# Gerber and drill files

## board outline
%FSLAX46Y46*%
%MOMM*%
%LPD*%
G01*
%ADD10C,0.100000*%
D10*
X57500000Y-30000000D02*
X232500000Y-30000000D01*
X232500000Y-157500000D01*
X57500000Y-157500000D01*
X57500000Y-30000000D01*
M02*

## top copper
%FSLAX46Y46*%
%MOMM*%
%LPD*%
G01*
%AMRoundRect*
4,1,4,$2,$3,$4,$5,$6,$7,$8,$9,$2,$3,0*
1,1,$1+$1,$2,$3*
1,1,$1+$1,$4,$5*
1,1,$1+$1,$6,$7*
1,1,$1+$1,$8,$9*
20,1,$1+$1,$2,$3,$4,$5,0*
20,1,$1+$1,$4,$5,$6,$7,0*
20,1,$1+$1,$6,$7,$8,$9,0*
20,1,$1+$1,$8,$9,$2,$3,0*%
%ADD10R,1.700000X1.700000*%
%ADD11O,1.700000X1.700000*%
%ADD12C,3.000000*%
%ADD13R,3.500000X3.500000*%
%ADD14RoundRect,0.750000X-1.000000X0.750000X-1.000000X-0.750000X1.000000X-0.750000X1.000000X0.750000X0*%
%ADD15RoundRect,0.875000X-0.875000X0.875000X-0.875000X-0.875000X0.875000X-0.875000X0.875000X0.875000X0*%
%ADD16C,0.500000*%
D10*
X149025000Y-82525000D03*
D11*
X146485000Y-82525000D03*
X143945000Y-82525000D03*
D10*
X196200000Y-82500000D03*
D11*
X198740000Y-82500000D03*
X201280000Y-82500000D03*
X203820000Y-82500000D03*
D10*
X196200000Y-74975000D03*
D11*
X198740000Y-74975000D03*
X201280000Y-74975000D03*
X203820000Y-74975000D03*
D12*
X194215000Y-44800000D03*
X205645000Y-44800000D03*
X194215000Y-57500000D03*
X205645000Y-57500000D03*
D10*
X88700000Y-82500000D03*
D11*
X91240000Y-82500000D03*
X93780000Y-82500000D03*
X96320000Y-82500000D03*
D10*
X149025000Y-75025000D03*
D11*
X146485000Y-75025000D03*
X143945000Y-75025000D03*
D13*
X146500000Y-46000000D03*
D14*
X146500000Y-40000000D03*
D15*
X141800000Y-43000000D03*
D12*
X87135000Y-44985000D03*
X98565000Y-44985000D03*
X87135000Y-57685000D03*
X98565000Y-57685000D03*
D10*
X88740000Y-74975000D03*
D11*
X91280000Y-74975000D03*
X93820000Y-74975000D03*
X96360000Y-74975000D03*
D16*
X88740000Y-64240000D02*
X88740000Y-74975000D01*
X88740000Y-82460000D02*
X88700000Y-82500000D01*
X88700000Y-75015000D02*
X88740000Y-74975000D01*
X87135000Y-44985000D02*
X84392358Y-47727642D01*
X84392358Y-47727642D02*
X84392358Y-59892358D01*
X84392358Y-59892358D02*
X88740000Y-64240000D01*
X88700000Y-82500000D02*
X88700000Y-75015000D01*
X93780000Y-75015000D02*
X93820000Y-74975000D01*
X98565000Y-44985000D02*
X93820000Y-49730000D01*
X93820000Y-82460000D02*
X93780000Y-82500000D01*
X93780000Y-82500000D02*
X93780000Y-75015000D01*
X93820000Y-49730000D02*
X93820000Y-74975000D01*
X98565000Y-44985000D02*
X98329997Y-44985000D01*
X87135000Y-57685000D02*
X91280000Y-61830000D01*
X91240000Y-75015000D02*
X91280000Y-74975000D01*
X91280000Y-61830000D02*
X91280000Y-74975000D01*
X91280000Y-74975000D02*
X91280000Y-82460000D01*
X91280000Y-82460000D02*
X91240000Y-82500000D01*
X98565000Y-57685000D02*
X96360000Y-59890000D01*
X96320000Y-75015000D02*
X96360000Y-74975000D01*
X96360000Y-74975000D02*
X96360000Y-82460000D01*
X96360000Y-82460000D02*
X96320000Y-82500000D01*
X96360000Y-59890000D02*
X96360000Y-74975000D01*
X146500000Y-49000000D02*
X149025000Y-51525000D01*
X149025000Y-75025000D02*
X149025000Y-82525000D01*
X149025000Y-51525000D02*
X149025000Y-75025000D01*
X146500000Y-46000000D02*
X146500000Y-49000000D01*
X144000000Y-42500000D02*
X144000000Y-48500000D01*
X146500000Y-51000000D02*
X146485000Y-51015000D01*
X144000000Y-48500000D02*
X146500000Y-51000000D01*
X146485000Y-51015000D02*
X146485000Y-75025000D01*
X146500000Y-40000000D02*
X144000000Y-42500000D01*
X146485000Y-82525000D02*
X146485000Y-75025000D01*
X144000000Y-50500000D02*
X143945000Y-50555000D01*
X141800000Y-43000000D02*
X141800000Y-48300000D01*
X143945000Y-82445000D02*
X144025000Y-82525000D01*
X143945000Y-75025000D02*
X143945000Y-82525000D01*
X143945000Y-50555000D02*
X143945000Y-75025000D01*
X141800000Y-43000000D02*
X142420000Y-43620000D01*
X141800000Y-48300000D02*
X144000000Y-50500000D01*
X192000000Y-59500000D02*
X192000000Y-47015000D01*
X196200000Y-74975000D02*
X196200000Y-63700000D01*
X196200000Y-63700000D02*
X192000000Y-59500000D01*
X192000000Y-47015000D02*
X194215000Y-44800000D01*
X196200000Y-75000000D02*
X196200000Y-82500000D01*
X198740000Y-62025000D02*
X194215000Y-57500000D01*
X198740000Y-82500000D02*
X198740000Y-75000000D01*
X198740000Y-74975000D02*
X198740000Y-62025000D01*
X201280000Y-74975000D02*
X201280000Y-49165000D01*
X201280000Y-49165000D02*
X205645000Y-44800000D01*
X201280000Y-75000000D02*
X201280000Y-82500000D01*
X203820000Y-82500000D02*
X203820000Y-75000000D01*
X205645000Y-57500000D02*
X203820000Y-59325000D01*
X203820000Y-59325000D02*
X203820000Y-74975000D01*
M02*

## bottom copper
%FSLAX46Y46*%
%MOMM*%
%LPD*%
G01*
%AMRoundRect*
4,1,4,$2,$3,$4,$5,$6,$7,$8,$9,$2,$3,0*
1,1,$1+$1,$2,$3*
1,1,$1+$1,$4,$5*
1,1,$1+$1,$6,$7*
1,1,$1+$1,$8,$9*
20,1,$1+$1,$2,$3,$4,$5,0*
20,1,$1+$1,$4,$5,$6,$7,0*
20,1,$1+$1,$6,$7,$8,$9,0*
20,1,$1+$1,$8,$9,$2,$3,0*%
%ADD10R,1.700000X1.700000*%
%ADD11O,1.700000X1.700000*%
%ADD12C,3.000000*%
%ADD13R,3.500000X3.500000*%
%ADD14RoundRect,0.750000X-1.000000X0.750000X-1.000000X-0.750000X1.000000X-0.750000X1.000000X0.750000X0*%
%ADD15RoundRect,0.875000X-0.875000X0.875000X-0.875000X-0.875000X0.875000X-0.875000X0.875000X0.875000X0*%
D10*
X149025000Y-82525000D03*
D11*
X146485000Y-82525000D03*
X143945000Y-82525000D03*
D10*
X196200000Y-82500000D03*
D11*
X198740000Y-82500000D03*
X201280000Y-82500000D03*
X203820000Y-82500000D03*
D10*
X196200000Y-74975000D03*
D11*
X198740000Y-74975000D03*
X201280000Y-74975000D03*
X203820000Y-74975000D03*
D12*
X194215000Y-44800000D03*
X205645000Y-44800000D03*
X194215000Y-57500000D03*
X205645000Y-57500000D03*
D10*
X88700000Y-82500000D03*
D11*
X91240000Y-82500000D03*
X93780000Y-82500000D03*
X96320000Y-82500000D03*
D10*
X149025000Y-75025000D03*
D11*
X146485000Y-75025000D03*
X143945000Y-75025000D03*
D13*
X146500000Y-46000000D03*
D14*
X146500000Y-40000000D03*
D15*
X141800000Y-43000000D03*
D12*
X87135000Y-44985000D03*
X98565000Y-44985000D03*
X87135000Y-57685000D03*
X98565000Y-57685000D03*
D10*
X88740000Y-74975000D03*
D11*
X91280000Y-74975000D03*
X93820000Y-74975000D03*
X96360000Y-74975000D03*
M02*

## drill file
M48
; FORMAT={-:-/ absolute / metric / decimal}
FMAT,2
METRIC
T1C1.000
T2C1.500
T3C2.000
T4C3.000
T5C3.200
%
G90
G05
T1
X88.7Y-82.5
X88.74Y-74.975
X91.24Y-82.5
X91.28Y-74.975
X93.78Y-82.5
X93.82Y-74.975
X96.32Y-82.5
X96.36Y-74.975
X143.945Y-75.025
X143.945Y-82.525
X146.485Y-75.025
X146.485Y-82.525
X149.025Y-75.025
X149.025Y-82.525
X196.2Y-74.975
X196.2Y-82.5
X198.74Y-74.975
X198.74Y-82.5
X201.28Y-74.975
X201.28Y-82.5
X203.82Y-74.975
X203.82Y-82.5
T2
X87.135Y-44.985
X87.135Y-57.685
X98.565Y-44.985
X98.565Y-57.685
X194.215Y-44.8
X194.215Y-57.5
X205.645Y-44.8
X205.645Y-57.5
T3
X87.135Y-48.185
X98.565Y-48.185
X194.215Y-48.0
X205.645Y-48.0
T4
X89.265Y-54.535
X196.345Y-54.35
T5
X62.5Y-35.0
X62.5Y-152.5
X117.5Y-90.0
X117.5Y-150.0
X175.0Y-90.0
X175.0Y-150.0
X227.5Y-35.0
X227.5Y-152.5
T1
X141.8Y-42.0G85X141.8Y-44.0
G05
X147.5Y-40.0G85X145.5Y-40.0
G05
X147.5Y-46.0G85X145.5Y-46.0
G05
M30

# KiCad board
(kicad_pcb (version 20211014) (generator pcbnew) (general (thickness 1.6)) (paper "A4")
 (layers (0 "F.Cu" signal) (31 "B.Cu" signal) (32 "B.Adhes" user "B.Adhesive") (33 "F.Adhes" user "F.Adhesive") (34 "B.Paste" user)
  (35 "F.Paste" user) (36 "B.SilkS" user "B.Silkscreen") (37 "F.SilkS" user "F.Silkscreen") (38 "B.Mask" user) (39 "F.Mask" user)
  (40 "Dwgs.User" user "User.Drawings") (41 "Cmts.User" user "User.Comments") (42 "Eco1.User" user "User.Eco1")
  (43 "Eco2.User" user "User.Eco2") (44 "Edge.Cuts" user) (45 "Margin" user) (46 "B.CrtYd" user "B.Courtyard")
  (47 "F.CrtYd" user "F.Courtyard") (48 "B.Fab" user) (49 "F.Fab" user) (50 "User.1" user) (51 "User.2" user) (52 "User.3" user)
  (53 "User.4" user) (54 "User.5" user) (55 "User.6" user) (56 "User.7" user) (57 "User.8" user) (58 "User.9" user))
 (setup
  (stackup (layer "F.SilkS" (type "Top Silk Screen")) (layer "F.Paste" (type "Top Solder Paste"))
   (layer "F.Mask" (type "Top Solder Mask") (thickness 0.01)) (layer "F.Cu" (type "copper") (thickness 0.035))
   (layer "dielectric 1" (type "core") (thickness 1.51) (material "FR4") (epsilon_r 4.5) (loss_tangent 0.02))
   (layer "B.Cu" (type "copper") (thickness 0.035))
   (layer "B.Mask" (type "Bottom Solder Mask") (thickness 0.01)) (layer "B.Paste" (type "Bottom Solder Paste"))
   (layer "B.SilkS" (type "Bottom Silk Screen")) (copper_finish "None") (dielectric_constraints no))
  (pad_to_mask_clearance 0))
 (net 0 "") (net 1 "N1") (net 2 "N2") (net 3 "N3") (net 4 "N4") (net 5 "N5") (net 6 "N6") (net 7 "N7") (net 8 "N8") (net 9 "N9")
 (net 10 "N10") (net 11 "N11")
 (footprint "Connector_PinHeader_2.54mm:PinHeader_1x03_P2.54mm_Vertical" (layer "F.Cu") (at 149.025 82.525 -90)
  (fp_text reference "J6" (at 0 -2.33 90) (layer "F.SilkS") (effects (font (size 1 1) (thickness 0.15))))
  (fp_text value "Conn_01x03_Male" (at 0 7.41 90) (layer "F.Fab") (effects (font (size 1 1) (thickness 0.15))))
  (pad "1" thru_hole rect (at 0 0 270) (size 1.7 1.7) (drill 1) (layers *.Cu *.Mask) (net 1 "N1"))
  (pad "2" thru_hole oval (at 0 2.54 270) (size 1.7 1.7) (drill 1) (layers *.Cu *.Mask) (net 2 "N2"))
  (pad "3" thru_hole oval (at 0 5.08 270) (size 1.7 1.7) (drill 1) (layers *.Cu *.Mask) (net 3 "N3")))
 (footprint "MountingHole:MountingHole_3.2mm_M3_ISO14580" (layer "F.Cu") (at 227.5 152.5)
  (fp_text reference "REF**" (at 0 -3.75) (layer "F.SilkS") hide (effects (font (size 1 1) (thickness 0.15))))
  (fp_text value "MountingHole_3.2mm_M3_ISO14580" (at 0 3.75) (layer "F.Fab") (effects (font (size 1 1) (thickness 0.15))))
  (pad "" np_thru_hole circle (at 0 0) (size 3.2 3.2) (drill 3.2) (layers *.Cu *.Mask)))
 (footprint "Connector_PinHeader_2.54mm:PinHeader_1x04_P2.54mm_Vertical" (layer "F.Cu") (at 196.2 82.5 90)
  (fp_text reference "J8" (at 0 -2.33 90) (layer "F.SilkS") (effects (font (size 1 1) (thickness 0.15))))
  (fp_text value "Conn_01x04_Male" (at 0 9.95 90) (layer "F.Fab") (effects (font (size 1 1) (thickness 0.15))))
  (pad "1" thru_hole rect (at 0 0 90) (size 1.7 1.7) (drill 1) (layers *.Cu *.Mask) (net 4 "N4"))
  (pad "2" thru_hole oval (at 0 2.54 90) (size 1.7 1.7) (drill 1) (layers *.Cu *.Mask) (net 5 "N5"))
  (pad "3" thru_hole oval (at 0 5.08 90) (size 1.7 1.7) (drill 1) (layers *.Cu *.Mask) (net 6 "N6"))
  (pad "4" thru_hole oval (at 0 7.62 90) (size 1.7 1.7) (drill 1) (layers *.Cu *.Mask) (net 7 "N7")))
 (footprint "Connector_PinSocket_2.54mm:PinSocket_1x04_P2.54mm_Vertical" (layer "F.Cu") (at 196.2 74.975 90)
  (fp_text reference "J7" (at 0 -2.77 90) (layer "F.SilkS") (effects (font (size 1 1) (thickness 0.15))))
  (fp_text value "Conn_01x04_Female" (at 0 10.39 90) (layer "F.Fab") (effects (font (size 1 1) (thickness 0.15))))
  (pad "1" thru_hole rect (at 0 0 90) (size 1.7 1.7) (drill 1) (layers *.Cu *.Mask) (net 4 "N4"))
  (pad "2" thru_hole oval (at 0 2.54 90) (size 1.7 1.7) (drill 1) (layers *.Cu *.Mask) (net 5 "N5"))
  (pad "3" thru_hole oval (at 0 5.08 90) (size 1.7 1.7) (drill 1) (layers *.Cu *.Mask) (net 6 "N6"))
  (pad "4" thru_hole oval (at 0 7.62 90) (size 1.7 1.7) (drill 1) (layers *.Cu *.Mask) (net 7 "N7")))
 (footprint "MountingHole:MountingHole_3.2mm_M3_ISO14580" (layer "F.Cu") (at 117.5 150)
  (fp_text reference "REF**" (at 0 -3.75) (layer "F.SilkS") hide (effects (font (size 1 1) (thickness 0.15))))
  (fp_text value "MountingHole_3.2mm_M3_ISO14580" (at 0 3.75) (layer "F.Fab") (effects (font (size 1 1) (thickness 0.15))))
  (pad "" np_thru_hole circle (at 0 0) (size 3.2 3.2) (drill 3.2) (layers *.Cu *.Mask)))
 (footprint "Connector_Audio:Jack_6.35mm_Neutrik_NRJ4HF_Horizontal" (layer "F.Cu") (at 194.215 57.5 90)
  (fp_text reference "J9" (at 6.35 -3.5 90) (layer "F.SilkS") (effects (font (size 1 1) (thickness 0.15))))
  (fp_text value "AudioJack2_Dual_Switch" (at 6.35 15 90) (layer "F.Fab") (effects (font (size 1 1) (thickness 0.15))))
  (pad "" np_thru_hole circle (at 3.15 2.13 90) (size 3 3) (drill 3) (layers *.Cu *.Mask))
  (pad "" np_thru_hole circle (at 9.5 0 90) (size 2 2) (drill 2) (layers *.Cu *.Mask))
  (pad "" np_thru_hole circle (at 9.5 11.43 90) (size 2 2) (drill 2) (layers *.Cu *.Mask))
  (pad "S" thru_hole circle (at 12.7 0 90) (size 3 3) (drill 1.5) (layers *.Cu *.Mask) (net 4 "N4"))
  (pad "SN" thru_hole circle (at 12.7 11.43 90) (size 3 3) (drill 1.5) (layers *.Cu *.Mask) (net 6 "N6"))
  (pad "T" thru_hole circle (at 0 0 90) (size 3 3) (drill 1.5) (layers *.Cu *.Mask) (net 5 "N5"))
  (pad "TN" thru_hole circle (at 0 11.43 90) (size 3 3) (drill 1.5) (layers *.Cu *.Mask) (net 7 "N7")))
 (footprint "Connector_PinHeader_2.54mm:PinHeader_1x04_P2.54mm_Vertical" (layer "F.Cu") (at 88.7 82.5 90)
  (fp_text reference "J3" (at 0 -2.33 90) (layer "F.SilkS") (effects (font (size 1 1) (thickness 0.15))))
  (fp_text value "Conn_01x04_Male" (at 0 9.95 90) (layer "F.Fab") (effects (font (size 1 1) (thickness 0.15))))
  (pad "1" thru_hole rect (at 0 0 90) (size 1.7 1.7) (drill 1) (layers *.Cu *.Mask) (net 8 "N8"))
  (pad "2" thru_hole oval (at 0 2.54 90) (size 1.7 1.7) (drill 1) (layers *.Cu *.Mask) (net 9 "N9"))
  (pad "3" thru_hole oval (at 0 5.08 90) (size 1.7 1.7) (drill 1) (layers *.Cu *.Mask) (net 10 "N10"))
  (pad "4" thru_hole oval (at 0 7.62 90) (size 1.7 1.7) (drill 1) (layers *.Cu *.Mask) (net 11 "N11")))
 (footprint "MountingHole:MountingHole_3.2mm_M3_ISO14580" (layer "F.Cu") (at 117.5 90)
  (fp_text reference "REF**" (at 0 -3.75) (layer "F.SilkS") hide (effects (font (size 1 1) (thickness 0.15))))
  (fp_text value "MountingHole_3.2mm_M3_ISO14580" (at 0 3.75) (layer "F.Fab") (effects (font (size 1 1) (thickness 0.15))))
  (pad "" np_thru_hole circle (at 0 0) (size 3.2 3.2) (drill 3.2) (layers *.Cu *.Mask)))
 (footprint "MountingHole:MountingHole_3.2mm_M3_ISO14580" (layer "F.Cu") (at 62.5 35)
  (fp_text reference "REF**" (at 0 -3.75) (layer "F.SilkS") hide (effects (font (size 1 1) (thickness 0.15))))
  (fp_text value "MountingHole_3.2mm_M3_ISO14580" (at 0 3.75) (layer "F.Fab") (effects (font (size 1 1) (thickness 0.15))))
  (pad "" np_thru_hole circle (at 0 0) (size 3.2 3.2) (drill 3.2) (layers *.Cu *.Mask)))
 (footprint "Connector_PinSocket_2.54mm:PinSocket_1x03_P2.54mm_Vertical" (layer "F.Cu") (at 149.025 75.025 -90)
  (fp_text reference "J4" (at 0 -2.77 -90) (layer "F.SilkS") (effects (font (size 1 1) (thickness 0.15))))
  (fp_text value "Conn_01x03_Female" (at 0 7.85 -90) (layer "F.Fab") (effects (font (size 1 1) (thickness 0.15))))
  (pad "1" thru_hole rect (at 0 0 270) (size 1.7 1.7) (drill 1) (layers *.Cu *.Mask) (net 1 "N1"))
  (pad "2" thru_hole oval (at 0 2.54 270) (size 1.7 1.7) (drill 1) (layers *.Cu *.Mask) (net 2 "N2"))
  (pad "3" thru_hole oval (at 0 5.08 270) (size 1.7 1.7) (drill 1) (layers *.Cu *.Mask) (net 3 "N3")))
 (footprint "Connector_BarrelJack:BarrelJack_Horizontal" (layer "F.Cu") (at 146.5 46 -90)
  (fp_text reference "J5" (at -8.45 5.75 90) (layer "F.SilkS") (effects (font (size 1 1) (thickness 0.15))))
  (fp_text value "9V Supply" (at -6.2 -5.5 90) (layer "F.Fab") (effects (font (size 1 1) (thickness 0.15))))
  (pad "1" thru_hole rect (at 0 0 270) (size 3.5 3.5) (drill oval 1 3) (layers *.Cu *.Mask) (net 1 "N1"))
  (pad "2" thru_hole roundrect (at -6 0 270) (size 3 3.5) (drill oval 1 3) (layers *.Cu *.Mask) (roundrect_rratio 0.25) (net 2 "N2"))
  (pad "3" thru_hole roundrect (at -3 4.7 270) (size 3.5 3.5) (drill oval 3 1) (layers *.Cu *.Mask) (roundrect_rratio 0.25) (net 3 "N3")))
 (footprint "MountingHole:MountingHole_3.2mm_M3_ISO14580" (layer "F.Cu") (at 175 90)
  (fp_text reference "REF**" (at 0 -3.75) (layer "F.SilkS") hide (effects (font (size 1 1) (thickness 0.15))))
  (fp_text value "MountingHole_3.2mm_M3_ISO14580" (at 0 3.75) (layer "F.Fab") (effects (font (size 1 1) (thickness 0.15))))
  (pad "" np_thru_hole circle (at 0 0) (size 3.2 3.2) (drill 3.2) (layers *.Cu *.Mask)))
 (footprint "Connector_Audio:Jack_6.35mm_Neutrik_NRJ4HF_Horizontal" (layer "F.Cu") (at 87.135 57.685 90)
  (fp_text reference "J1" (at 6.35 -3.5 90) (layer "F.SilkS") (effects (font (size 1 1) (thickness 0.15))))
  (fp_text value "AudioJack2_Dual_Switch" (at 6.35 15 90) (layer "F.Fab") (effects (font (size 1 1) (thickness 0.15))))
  (pad "" np_thru_hole circle (at 3.15 2.13 90) (size 3 3) (drill 3) (layers *.Cu *.Mask))
  (pad "" np_thru_hole circle (at 9.5 11.43 90) (size 2 2) (drill 2) (layers *.Cu *.Mask))
  (pad "" np_thru_hole circle (at 9.5 0 90) (size 2 2) (drill 2) (layers *.Cu *.Mask))
  (pad "S" thru_hole circle (at 12.7 0 90) (size 3 3) (drill 1.5) (layers *.Cu *.Mask) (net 8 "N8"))
  (pad "SN" thru_hole circle (at 12.7 11.43 90) (size 3 3) (drill 1.5) (layers *.Cu *.Mask) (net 10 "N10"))
  (pad "T" thru_hole circle (at 0 0 90) (size 3 3) (drill 1.5) (layers *.Cu *.Mask) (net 9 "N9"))
  (pad "TN" thru_hole circle (at 0 11.43 90) (size 3 3) (drill 1.5) (layers *.Cu *.Mask) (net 11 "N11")))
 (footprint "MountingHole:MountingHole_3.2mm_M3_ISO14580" (layer "F.Cu") (at 62.5 152.5)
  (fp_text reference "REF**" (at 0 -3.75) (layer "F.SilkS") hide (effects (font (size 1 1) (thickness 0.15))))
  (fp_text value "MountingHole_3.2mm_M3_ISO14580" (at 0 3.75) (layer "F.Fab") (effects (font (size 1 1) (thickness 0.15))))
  (pad "" np_thru_hole circle (at 0 0) (size 3.2 3.2) (drill 3.2) (layers *.Cu *.Mask)))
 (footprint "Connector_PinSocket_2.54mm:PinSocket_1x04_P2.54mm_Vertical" (layer "F.Cu") (at 88.74 74.975 90)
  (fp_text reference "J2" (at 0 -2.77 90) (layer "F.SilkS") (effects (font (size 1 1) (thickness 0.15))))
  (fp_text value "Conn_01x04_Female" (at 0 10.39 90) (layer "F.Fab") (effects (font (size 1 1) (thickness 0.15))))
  (pad "1" thru_hole rect (at 0 0 90) (size 1.7 1.7) (drill 1) (layers *.Cu *.Mask) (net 8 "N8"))
  (pad "2" thru_hole oval (at 0 2.54 90) (size 1.7 1.7) (drill 1) (layers *.Cu *.Mask) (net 9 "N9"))
  (pad "3" thru_hole oval (at 0 5.08 90) (size 1.7 1.7) (drill 1) (layers *.Cu *.Mask) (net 10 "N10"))
  (pad "4" thru_hole oval (at 0 7.62 90) (size 1.7 1.7) (drill 1) (layers *.Cu *.Mask) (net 11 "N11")))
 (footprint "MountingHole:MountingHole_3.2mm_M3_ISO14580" (layer "F.Cu") (at 175 150)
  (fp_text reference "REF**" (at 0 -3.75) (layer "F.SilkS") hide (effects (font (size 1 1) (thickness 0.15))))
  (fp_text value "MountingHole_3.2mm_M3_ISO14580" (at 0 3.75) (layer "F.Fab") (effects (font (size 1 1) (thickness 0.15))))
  (pad "" np_thru_hole circle (at 0 0) (size 3.2 3.2) (drill 3.2) (layers *.Cu *.Mask)))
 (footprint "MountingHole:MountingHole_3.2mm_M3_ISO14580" (layer "F.Cu") (at 227.5 35)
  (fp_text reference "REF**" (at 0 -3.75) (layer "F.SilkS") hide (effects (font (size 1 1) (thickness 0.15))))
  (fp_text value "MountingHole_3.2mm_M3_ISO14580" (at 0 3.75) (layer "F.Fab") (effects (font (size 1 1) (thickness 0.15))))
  (pad "" np_thru_hole circle (at 0 0) (size 3.2 3.2) (drill 3.2) (layers *.Cu *.Mask)))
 (gr_rect (start 57.5 30) (end 232.5 157.5) (layer "Edge.Cuts") (width 0.1) (fill none))
 (segment (start 88.74 64.24) (end 88.74 74.975) (width 0.5) (layer "F.Cu") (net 8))
 (segment (start 88.74 82.46) (end 88.7 82.5) (width 0.5) (layer "F.Cu") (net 8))
 (segment (start 88.7 75.015) (end 88.74 74.975) (width 0.5) (layer "F.Cu") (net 8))
 (segment (start 87.135 44.985) (end 84.392358 47.727642) (width 0.5) (layer "F.Cu") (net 8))
 (segment (start 84.392358 47.727642) (end 84.392358 59.892358) (width 0.5) (layer "F.Cu") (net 8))
 (segment (start 84.392358 59.892358) (end 88.74 64.24) (width 0.5) (layer "F.Cu") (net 8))
 (segment (start 88.7 82.5) (end 88.7 75.015) (width 0.5) (layer "F.Cu") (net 8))
 (segment (start 93.78 75.015) (end 93.82 74.975) (width 0.5) (layer "F.Cu") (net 10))
 (segment (start 98.565 44.985) (end 93.82 49.73) (width 0.5) (layer "F.Cu") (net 10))
 (segment (start 93.82 82.46) (end 93.78 82.5) (width 0.5) (layer "F.Cu") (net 10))
 (segment (start 93.78 82.5) (end 93.78 75.015) (width 0.5) (layer "F.Cu") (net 10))
 (segment (start 93.82 49.73) (end 93.82 74.975) (width 0.5) (layer "F.Cu") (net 10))
 (segment (start 98.565 44.985) (end 98.329997 44.985) (width 0.5) (layer "F.Cu") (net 10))
 (segment (start 87.135 57.685) (end 91.28 61.83) (width 0.5) (layer "F.Cu") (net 9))
 (segment (start 91.24 75.015) (end 91.28 74.975) (width 0.5) (layer "F.Cu") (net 9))
 (segment (start 91.28 61.83) (end 91.28 74.975) (width 0.5) (layer "F.Cu") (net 9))
 (segment (start 91.28 74.975) (end 91.28 82.46) (width 0.5) (layer "F.Cu") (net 9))
 (segment (start 91.28 82.46) (end 91.24 82.5) (width 0.5) (layer "F.Cu") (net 9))
 (segment (start 98.565 57.685) (end 96.36 59.89) (width 0.5) (layer "F.Cu") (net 11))
 (segment (start 96.32 75.015) (end 96.36 74.975) (width 0.5) (layer "F.Cu") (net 11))
 (segment (start 96.36 74.975) (end 96.36 82.46) (width 0.5) (layer "F.Cu") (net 11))
 (segment (start 96.36 82.46) (end 96.32 82.5) (width 0.5) (layer "F.Cu") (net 11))
 (segment (start 96.36 59.89) (end 96.36 74.975) (width 0.5) (layer "F.Cu") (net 11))
 (segment (start 146.5 49) (end 149.025 51.525) (width 0.5) (layer "F.Cu") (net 1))
 (segment (start 149.025 75.025) (end 149.025 82.525) (width 0.5) (layer "F.Cu") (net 1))
 (segment (start 149.025 51.525) (end 149.025 75.025) (width 0.5) (layer "F.Cu") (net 1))
 (segment (start 146.5 46) (end 146.5 49) (width 0.5) (layer "F.Cu") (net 1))
 (segment (start 144 42.5) (end 144 48.5) (width 0.5) (layer "F.Cu") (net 2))
 (segment (start 146.5 51) (end 146.485 51.015) (width 0.5) (layer "F.Cu") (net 2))
 (segment (start 144 48.5) (end 146.5 51) (width 0.5) (layer "F.Cu") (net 2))
 (segment (start 146.485 51.015) (end 146.485 75.025) (width 0.5) (layer "F.Cu") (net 2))
 (segment (start 146.5 40) (end 144 42.5) (width 0.5) (layer "F.Cu") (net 2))
 (segment (start 146.485 82.525) (end 146.485 75.025) (width 0.5) (layer "F.Cu") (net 2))
 (segment (start 144 50.5) (end 143.945 50.555) (width 0.5) (layer "F.Cu") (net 3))
 (segment (start 141.8 43) (end 141.8 48.3) (width 0.5) (layer "F.Cu") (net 3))
 (segment (start 143.945 82.445) (end 144.025 82.525) (width 0.5) (layer "F.Cu") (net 3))
 (segment (start 143.945 75.025) (end 143.945 82.525) (width 0.5) (layer "F.Cu") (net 3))
 (segment (start 143.945 50.555) (end 143.945 75.025) (width 0.5) (layer "F.Cu") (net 3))
 (segment (start 141.8 43) (end 142.42 43.62) (width 0.5) (layer "F.Cu") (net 3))
 (segment (start 141.8 48.3) (end 144 50.5) (width 0.5) (layer "F.Cu") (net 3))
 (segment (start 192 59.5) (end 192 47.015) (width 0.5) (layer "F.Cu") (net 4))
 (segment (start 196.2 74.975) (end 196.2 63.7) (width 0.5) (layer "F.Cu") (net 4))
 (segment (start 196.2 63.7) (end 192 59.5) (width 0.5) (layer "F.Cu") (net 4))
 (segment (start 192 47.015) (end 194.215 44.8) (width 0.5) (layer "F.Cu") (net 4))
 (segment (start 196.2 75) (end 196.2 82.5) (width 0.5) (layer "F.Cu") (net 4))
 (segment (start 198.74 62.025) (end 194.215 57.5) (width 0.5) (layer "F.Cu") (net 5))
 (segment (start 198.74 82.5) (end 198.74 75) (width 0.5) (layer "F.Cu") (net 5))
 (segment (start 198.74 74.975) (end 198.74 62.025) (width 0.5) (layer "F.Cu") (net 5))
 (segment (start 201.28 74.975) (end 201.28 49.165) (width 0.5) (layer "F.Cu") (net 6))
 (segment (start 201.28 49.165) (end 205.645 44.8) (width 0.5) (layer "F.Cu") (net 6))
 (segment (start 201.28 75) (end 201.28 82.5) (width 0.5) (layer "F.Cu") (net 6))
 (segment (start 203.82 82.5) (end 203.82 75) (width 0.5) (layer "F.Cu") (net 7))
 (segment (start 205.645 57.5) (end 203.82 59.325) (width 0.5) (layer "F.Cu") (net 7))
 (segment (start 203.82 59.325) (end 203.82 74.975) (width 0.5) (layer "F.Cu") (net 7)))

